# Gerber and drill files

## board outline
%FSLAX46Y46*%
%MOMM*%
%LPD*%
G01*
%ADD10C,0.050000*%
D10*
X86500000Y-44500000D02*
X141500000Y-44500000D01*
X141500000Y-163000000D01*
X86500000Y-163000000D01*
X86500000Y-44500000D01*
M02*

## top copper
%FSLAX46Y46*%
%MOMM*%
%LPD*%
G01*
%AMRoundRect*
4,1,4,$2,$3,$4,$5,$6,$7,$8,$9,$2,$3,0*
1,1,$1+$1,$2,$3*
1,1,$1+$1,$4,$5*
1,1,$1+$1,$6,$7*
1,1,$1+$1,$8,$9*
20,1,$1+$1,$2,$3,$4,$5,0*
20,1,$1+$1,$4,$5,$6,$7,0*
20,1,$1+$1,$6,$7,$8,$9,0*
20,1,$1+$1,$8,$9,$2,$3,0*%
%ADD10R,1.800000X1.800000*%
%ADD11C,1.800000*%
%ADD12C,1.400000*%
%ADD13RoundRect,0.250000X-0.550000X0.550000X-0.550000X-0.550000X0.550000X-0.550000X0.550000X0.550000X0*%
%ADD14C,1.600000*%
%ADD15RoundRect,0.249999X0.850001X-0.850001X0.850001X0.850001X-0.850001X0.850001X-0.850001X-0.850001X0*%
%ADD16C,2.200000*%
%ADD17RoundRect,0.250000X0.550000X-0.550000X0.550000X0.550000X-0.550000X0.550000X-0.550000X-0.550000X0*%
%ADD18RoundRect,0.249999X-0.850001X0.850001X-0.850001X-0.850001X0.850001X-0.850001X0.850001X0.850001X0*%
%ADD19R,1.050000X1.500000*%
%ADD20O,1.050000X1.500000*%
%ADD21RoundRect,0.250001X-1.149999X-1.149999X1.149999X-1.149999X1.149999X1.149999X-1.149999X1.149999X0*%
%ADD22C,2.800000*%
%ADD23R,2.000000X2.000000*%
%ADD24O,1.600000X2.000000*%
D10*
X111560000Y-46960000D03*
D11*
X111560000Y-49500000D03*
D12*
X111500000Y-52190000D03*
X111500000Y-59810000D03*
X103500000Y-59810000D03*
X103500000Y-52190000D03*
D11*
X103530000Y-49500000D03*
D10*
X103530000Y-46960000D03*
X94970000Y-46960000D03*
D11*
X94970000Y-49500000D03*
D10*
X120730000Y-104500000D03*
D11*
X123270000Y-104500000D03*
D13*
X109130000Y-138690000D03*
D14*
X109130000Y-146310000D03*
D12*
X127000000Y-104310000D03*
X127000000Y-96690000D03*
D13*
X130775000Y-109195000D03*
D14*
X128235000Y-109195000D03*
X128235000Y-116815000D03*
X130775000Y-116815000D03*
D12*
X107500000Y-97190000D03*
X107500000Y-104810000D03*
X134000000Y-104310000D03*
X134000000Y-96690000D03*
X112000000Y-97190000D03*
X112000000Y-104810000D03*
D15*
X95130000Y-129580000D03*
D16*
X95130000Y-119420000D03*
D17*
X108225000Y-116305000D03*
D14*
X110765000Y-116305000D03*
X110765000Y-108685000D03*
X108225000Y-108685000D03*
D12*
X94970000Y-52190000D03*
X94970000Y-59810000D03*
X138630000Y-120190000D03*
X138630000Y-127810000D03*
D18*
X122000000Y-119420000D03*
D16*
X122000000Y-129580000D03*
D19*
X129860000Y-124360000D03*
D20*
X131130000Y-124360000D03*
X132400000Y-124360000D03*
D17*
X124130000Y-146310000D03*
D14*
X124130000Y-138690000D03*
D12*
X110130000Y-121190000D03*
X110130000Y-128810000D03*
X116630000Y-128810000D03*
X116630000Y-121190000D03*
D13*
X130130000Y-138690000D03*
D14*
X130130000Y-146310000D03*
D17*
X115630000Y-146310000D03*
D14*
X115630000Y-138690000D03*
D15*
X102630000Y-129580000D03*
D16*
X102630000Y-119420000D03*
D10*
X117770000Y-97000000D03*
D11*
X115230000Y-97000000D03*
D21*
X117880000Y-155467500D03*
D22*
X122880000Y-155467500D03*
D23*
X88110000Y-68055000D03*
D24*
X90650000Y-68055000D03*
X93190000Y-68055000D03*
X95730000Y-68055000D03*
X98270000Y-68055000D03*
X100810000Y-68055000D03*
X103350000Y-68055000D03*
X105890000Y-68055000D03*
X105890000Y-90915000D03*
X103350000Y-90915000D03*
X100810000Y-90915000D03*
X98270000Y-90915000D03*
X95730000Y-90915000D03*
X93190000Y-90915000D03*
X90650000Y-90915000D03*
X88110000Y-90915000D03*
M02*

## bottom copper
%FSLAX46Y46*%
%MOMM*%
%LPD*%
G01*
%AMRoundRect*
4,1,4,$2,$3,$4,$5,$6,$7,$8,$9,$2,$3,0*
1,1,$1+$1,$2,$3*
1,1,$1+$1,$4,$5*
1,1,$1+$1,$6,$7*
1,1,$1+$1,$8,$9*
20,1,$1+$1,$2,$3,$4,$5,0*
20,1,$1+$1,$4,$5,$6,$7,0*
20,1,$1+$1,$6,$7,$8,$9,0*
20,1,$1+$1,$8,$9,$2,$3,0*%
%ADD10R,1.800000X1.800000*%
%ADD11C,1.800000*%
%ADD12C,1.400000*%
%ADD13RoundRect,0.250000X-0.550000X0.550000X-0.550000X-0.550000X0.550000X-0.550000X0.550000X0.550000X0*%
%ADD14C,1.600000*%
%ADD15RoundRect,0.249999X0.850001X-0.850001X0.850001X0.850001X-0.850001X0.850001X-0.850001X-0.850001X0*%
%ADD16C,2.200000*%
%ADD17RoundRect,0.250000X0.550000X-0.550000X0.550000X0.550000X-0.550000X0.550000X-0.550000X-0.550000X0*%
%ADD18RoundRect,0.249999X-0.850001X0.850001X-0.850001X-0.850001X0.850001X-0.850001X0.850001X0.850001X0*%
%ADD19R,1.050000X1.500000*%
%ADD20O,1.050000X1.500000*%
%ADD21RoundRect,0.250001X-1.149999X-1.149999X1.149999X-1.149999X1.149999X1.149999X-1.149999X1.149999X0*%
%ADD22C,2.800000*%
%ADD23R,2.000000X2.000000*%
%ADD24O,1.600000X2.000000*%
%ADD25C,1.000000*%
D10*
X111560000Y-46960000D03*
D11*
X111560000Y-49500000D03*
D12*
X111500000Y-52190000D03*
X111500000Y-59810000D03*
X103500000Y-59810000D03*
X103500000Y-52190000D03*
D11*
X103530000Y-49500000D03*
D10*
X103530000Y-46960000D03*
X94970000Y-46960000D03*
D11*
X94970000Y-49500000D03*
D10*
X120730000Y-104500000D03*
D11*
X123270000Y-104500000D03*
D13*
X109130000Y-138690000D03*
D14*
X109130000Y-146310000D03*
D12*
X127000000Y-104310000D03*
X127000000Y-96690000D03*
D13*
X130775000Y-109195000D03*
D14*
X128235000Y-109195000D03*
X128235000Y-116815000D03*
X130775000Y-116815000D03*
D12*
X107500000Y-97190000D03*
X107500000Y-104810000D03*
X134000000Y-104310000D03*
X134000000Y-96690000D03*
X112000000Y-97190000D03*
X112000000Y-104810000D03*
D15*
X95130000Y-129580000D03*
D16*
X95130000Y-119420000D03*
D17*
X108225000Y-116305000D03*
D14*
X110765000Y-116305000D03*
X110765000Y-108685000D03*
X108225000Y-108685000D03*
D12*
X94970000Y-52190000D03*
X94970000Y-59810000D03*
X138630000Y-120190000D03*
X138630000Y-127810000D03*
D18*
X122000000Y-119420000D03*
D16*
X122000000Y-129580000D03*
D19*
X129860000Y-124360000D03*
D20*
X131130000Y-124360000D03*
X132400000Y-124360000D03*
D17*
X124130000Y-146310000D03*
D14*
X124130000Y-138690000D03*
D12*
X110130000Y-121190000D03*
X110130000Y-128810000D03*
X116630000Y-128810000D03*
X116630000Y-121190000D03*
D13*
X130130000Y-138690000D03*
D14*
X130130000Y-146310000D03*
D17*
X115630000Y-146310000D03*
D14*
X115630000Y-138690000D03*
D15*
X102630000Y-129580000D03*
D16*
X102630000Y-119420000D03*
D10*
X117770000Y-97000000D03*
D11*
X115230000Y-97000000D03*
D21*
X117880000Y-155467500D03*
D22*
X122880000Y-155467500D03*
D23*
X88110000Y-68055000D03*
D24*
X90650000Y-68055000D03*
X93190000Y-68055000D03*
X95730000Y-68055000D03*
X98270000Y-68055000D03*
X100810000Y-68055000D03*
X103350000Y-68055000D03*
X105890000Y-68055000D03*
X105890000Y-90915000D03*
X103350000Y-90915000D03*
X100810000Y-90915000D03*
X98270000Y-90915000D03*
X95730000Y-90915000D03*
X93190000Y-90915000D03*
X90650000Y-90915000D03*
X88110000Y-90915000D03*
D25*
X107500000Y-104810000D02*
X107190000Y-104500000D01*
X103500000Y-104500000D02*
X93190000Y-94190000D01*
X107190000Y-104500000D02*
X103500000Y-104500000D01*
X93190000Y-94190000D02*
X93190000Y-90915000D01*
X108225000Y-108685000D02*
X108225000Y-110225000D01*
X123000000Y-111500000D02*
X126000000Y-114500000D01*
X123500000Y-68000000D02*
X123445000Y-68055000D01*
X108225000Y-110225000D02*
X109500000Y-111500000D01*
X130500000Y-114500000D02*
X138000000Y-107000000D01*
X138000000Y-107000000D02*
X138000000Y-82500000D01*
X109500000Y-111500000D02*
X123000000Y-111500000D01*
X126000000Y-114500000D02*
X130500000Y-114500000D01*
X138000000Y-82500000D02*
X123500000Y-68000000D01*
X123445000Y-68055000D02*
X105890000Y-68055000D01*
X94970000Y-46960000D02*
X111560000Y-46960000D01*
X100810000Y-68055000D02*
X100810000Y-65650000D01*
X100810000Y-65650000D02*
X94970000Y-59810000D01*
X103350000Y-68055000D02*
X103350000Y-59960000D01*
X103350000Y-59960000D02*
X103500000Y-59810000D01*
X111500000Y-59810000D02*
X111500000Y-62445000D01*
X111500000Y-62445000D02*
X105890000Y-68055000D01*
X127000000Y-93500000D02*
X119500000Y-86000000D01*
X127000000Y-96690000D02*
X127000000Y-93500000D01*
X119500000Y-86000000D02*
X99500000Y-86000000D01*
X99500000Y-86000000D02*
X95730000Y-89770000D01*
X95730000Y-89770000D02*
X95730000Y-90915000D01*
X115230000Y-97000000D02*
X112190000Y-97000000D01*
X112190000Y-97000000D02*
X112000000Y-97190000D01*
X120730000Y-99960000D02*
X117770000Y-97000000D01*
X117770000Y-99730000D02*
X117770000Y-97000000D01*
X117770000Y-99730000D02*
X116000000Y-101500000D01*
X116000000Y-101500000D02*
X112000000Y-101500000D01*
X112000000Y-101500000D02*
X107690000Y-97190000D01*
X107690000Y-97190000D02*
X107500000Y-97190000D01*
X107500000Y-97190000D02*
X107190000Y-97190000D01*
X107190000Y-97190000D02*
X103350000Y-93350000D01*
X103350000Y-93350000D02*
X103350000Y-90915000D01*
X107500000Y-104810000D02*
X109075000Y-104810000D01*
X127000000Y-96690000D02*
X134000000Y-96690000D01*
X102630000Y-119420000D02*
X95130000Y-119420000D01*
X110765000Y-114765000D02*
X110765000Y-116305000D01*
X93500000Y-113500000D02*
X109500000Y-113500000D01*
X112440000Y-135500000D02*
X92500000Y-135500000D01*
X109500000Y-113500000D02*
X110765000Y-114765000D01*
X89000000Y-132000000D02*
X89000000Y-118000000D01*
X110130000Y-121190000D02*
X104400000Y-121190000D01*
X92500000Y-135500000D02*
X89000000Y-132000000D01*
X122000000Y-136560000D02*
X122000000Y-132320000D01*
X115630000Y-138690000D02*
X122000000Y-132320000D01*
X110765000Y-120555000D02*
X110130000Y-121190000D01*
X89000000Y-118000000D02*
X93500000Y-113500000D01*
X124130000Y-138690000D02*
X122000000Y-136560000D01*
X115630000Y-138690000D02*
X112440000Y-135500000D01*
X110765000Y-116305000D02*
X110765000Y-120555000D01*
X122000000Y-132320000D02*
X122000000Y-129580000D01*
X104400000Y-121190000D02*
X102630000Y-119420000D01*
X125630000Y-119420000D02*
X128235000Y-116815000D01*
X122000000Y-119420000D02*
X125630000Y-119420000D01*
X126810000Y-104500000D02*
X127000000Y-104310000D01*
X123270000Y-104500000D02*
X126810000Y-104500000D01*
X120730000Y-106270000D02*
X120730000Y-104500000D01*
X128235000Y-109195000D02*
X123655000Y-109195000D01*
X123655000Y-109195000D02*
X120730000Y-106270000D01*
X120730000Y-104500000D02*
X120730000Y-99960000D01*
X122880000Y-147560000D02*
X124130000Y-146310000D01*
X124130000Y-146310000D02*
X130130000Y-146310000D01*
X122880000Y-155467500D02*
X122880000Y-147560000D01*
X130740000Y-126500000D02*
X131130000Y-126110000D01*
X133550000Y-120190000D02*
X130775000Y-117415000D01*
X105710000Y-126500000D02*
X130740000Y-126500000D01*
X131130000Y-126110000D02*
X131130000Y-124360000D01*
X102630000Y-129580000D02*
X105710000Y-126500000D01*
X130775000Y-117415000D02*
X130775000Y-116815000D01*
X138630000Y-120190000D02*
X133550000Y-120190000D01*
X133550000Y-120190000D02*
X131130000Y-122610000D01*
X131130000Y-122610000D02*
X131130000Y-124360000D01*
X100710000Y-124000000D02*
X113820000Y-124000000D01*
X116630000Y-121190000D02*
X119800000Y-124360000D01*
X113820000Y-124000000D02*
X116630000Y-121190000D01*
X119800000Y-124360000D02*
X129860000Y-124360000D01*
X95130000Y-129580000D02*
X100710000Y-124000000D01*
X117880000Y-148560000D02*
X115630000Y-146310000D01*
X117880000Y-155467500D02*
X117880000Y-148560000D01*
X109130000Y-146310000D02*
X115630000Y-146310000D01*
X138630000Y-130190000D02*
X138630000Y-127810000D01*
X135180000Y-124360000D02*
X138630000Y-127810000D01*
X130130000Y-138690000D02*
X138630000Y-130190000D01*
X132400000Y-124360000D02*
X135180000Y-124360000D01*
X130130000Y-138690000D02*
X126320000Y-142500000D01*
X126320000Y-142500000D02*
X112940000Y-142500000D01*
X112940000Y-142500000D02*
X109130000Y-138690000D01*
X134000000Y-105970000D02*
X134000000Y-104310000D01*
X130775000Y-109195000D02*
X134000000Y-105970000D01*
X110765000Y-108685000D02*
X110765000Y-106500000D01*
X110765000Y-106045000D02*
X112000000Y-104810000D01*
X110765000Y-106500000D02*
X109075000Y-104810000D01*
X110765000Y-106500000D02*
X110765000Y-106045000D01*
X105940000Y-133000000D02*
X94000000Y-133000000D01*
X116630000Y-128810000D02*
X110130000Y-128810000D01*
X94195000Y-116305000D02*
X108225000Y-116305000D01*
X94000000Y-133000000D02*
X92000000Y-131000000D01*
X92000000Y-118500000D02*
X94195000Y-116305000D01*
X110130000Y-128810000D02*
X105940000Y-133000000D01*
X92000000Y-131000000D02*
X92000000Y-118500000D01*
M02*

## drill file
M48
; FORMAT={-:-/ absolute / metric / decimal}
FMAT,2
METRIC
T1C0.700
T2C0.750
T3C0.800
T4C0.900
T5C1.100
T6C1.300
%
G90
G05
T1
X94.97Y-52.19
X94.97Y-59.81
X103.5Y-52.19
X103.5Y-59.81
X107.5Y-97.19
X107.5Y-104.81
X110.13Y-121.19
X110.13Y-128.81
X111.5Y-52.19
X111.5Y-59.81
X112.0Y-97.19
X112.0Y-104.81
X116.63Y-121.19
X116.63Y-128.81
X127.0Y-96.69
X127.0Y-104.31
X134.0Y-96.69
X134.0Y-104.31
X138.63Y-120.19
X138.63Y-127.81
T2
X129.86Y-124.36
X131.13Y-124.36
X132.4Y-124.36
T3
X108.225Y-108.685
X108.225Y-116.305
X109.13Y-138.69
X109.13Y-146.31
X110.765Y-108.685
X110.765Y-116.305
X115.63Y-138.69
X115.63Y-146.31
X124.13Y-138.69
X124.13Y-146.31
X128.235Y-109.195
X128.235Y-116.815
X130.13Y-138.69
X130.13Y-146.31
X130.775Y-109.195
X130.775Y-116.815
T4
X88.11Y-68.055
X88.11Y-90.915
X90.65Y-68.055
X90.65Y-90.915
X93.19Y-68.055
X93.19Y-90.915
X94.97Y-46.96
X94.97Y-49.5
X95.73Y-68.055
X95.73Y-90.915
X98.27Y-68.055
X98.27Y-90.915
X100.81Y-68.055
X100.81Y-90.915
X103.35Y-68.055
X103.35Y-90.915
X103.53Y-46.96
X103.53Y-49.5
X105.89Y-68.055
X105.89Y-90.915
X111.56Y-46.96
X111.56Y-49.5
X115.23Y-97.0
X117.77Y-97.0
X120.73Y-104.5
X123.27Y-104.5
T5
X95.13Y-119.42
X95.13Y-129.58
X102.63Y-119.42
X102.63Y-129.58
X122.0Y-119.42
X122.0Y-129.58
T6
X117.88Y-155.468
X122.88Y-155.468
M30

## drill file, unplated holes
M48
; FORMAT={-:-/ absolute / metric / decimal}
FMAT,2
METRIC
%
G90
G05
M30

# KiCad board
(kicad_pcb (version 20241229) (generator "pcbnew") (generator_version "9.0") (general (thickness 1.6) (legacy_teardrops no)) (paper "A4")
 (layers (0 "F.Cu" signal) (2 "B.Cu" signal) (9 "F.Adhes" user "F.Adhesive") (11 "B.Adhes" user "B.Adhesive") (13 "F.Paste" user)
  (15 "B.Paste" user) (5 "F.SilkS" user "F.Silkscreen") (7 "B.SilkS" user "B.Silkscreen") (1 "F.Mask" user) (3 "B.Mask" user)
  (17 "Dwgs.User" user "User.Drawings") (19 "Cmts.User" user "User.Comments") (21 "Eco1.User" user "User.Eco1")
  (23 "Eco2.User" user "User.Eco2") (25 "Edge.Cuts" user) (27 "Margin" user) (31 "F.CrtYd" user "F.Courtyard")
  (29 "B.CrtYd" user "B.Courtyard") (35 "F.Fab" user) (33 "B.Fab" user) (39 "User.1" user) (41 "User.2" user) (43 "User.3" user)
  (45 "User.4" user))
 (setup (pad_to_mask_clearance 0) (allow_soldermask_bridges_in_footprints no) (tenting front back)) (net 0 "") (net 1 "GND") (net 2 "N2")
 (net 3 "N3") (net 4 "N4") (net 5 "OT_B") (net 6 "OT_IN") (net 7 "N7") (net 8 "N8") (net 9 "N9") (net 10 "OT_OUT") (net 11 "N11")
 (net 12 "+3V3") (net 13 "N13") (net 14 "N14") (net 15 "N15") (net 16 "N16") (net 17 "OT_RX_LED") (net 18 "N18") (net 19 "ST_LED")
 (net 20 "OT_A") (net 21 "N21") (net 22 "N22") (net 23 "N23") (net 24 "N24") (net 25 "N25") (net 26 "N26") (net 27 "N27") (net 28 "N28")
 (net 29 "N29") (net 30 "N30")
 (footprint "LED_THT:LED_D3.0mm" (layer "F.Cu") (at 94.97 46.96 -90)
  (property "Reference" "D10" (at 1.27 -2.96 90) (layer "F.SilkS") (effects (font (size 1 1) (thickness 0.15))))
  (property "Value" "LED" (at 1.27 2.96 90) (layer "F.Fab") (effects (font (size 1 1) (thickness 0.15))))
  (pad "1" thru_hole rect (at 0 0 270) (size 1.8 1.8) (drill 0.9) (layers "*.Cu" "*.Mask") (remove_unused_layers no) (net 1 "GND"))
  (pad "2" thru_hole circle (at 2.54 0 270) (size 1.8 1.8) (drill 0.9) (layers "*.Cu" "*.Mask") (remove_unused_layers no) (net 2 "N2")))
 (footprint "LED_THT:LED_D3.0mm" (layer "F.Cu") (at 120.73 104.5)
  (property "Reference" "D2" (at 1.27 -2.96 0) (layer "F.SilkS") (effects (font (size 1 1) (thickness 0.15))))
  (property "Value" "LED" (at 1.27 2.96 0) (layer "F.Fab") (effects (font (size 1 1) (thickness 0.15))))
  (pad "1" thru_hole rect (at 0 0) (size 1.8 1.8) (drill 0.9) (layers "*.Cu" "*.Mask") (remove_unused_layers no) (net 1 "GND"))
  (pad "2" thru_hole circle (at 2.54 0) (size 1.8 1.8) (drill 0.9) (layers "*.Cu" "*.Mask") (remove_unused_layers no) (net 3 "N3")))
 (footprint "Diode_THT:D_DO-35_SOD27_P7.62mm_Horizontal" (layer "F.Cu") (at 109.13 138.69 -90)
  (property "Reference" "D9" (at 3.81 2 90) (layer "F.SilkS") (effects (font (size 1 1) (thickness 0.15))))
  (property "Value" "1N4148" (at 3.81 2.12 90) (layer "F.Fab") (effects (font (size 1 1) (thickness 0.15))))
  (pad "1" thru_hole roundrect (at 0 0 270) (size 1.6 1.6) (drill 0.8) (layers "*.Cu" "*.Mask") (remove_unused_layers no)
   (roundrect_rratio 0.15625) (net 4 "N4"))
  (pad "2" thru_hole circle (at 7.62 0 270) (size 1.6 1.6) (drill 0.8) (layers "*.Cu" "*.Mask") (remove_unused_layers no) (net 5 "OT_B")))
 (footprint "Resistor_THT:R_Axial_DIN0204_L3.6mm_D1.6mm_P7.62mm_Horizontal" (layer "F.Cu") (at 127 104.31 90)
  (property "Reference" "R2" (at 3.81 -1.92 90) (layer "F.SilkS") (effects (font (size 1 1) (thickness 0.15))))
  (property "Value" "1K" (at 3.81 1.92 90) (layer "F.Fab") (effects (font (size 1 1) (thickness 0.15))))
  (pad "1" thru_hole circle (at 0 0 90) (size 1.4 1.4) (drill 0.7) (layers "*.Cu" "*.Mask") (remove_unused_layers no) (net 3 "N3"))
  (pad "2" thru_hole circle (at 7.62 0 90) (size 1.4 1.4) (drill 0.7) (layers "*.Cu" "*.Mask") (remove_unused_layers no) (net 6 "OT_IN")))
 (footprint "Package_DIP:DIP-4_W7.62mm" (layer "F.Cu") (at 130.775 109.195 -90)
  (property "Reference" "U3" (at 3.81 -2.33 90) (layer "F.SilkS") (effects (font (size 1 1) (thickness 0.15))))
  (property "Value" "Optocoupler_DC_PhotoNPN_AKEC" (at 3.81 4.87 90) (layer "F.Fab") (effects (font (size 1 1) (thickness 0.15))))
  (pad "1" thru_hole roundrect (at 0 0 270) (size 1.6 1.6) (drill 0.8) (layers "*.Cu" "*.Mask") (remove_unused_layers no)
   (roundrect_rratio 0.15625) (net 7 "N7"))
  (pad "2" thru_hole circle (at 0 2.54 270) (size 1.6 1.6) (drill 0.8) (layers "*.Cu" "*.Mask") (remove_unused_layers no) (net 1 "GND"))
  (pad "3" thru_hole circle (at 7.62 2.54 270) (size 1.6 1.6) (drill 0.8) (layers "*.Cu" "*.Mask") (remove_unused_layers no) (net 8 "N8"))
  (pad "4" thru_hole circle (at 7.62 0 270) (size 1.6 1.6) (drill 0.8) (layers "*.Cu" "*.Mask") (remove_unused_layers no) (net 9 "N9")))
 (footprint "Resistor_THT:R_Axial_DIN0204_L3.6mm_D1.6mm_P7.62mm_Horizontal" (layer "F.Cu") (at 107.5 97.19 -90)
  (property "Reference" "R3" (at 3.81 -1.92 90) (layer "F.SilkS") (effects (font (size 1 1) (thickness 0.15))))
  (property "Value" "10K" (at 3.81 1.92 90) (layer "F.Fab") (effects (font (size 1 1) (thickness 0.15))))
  (pad "1" thru_hole circle (at 0 0 270) (size 1.4 1.4) (drill 0.7) (layers "*.Cu" "*.Mask") (remove_unused_layers no) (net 1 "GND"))
  (pad "2" thru_hole circle (at 7.62 0 270) (size 1.4 1.4) (drill 0.7) (layers "*.Cu" "*.Mask") (remove_unused_layers no) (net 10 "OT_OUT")))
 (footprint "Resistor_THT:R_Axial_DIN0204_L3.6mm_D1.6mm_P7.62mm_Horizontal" (layer "F.Cu") (at 134 104.31 90)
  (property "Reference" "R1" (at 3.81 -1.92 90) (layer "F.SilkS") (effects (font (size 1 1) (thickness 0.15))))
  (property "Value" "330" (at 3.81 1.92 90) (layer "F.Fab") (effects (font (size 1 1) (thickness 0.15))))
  (pad "1" thru_hole circle (at 0 0 90) (size 1.4 1.4) (drill 0.7) (layers "*.Cu" "*.Mask") (remove_unused_layers no) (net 7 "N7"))
  (pad "2" thru_hole circle (at 7.62 0 90) (size 1.4 1.4) (drill 0.7) (layers "*.Cu" "*.Mask") (remove_unused_layers no) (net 6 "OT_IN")))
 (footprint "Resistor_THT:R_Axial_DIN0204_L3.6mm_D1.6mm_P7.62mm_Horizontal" (layer "F.Cu") (at 111.5 52.19 -90)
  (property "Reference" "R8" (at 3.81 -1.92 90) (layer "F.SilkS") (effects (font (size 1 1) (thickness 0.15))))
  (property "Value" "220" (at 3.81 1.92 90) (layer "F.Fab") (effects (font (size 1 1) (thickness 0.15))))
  (pad "1" thru_hole circle (at 0 0 270) (size 1.4 1.4) (drill 0.7) (layers "*.Cu" "*.Mask") (remove_unused_layers no) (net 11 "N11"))
  (pad "2" thru_hole circle (at 7.62 0 270) (size 1.4 1.4) (drill 0.7) (layers "*.Cu" "*.Mask") (remove_unused_layers no) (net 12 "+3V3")))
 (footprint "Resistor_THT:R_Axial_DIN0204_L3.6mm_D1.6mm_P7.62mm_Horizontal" (layer "F.Cu") (at 112 97.19 -90)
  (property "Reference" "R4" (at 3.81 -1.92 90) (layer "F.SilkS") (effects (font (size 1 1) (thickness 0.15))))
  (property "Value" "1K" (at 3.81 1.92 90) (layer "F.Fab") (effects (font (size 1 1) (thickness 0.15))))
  (pad "1" thru_hole circle (at 0 0 270) (size 1.4 1.4) (drill 0.7) (layers "*.Cu" "*.Mask") (remove_unused_layers no) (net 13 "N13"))
  (pad "2" thru_hole circle (at 7.62 0 270) (size 1.4 1.4) (drill 0.7) (layers "*.Cu" "*.Mask") (remove_unused_layers no) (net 10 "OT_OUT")))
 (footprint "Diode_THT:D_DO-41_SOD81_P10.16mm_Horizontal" (layer "F.Cu") (at 95.13 129.58 90)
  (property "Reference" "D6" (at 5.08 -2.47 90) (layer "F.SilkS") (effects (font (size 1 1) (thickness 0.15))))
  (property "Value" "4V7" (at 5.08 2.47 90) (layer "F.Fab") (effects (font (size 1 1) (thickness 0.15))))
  (pad "1" thru_hole roundrect (at 0 0 90) (size 2.2 2.2) (drill 1.1) (layers "*.Cu" "*.Mask") (remove_unused_layers no)
   (roundrect_rratio 0.113636) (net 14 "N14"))
  (pad "2" thru_hole circle (at 10.16 0 90) (size 2.2 2.2) (drill 1.1) (layers "*.Cu" "*.Mask") (remove_unused_layers no) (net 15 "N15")))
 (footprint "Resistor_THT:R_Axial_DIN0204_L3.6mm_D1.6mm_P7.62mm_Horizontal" (layer "F.Cu") (at 103.5 52.19 -90)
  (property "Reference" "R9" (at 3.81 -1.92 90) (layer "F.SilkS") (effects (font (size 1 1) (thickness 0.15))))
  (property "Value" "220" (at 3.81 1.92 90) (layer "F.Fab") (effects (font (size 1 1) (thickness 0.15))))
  (pad "1" thru_hole circle (at 0 0 270) (size 1.4 1.4) (drill 0.7) (layers "*.Cu" "*.Mask") (remove_unused_layers no) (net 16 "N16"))
  (pad "2" thru_hole circle (at 7.62 0 270) (size 1.4 1.4) (drill 0.7) (layers "*.Cu" "*.Mask") (remove_unused_layers no)
   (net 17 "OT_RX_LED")))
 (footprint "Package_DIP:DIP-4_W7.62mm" (layer "F.Cu") (at 108.225 116.305 90)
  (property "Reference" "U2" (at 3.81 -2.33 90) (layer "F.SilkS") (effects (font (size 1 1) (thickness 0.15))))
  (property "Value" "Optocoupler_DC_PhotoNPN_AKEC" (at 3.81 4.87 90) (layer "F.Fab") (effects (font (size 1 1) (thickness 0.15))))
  (pad "1" thru_hole roundrect (at 0 0 90) (size 1.6 1.6) (drill 0.8) (layers "*.Cu" "*.Mask") (remove_unused_layers no)
   (roundrect_rratio 0.15625) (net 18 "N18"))
  (pad "2" thru_hole circle (at 0 2.54 90) (size 1.6 1.6) (drill 0.8) (layers "*.Cu" "*.Mask") (remove_unused_layers no) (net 15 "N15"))
  (pad "3" thru_hole circle (at 7.62 2.54 90) (size 1.6 1.6) (drill 0.8) (layers "*.Cu" "*.Mask") (remove_unused_layers no)
   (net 10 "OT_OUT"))
  (pad "4" thru_hole circle (at 7.62 0 90) (size 1.6 1.6) (drill 0.8) (layers "*.Cu" "*.Mask") (remove_unused_layers no) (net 12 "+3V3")))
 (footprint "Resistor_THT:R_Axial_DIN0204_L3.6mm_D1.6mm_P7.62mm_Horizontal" (layer "F.Cu") (at 94.97 52.19 -90)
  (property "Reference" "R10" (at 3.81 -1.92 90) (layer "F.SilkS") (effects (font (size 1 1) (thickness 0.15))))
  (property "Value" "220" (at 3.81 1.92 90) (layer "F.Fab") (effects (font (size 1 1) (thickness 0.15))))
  (pad "1" thru_hole circle (at 0 0 270) (size 1.4 1.4) (drill 0.7) (layers "*.Cu" "*.Mask") (remove_unused_layers no) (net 2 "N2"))
  (pad "2" thru_hole circle (at 7.62 0 270) (size 1.4 1.4) (drill 0.7) (layers "*.Cu" "*.Mask") (remove_unused_layers no) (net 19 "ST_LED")))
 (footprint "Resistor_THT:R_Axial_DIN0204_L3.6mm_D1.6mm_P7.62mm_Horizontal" (layer "F.Cu") (at 138.63 120.19 -90)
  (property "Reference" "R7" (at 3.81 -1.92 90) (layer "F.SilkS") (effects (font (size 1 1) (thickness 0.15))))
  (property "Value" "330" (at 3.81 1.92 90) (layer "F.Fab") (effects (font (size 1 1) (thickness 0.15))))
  (pad "1" thru_hole circle (at 0 0 270) (size 1.4 1.4) (drill 0.7) (layers "*.Cu" "*.Mask") (remove_unused_layers no) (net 9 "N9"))
  (pad "2" thru_hole circle (at 7.62 0 270) (size 1.4 1.4) (drill 0.7) (layers "*.Cu" "*.Mask") (remove_unused_layers no) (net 4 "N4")))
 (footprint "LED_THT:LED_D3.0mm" (layer "F.Cu") (at 111.56 46.96 -90)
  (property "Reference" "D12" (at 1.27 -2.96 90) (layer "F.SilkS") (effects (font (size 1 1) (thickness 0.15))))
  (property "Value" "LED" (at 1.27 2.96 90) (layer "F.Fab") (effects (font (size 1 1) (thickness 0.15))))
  (pad "1" thru_hole rect (at 0 0 270) (size 1.8 1.8) (drill 0.9) (layers "*.Cu" "*.Mask") (remove_unused_layers no) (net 1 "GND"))
  (pad "2" thru_hole circle (at 2.54 0 270) (size 1.8 1.8) (drill 0.9) (layers "*.Cu" "*.Mask") (remove_unused_layers no) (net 11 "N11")))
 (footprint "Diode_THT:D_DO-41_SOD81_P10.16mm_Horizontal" (layer "F.Cu") (at 122 119.42 -90)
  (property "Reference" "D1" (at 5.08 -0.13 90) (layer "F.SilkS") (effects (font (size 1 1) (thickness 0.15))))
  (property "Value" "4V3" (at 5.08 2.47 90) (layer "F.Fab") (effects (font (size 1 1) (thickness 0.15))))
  (pad "1" thru_hole roundrect (at 0 0 270) (size 2.2 2.2) (drill 1.1) (layers "*.Cu" "*.Mask") (remove_unused_layers no)
   (roundrect_rratio 0.113636) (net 8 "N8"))
  (pad "2" thru_hole circle (at 10.16 0 270) (size 2.2 2.2) (drill 1.1) (layers "*.Cu" "*.Mask") (remove_unused_layers no) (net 15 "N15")))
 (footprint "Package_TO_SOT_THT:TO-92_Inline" (layer "F.Cu") (at 129.86 124.36)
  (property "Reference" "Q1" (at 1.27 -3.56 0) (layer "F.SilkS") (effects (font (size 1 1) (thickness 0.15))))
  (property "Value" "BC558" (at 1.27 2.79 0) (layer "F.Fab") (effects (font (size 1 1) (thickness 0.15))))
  (pad "1" thru_hole rect (at 0 0) (size 1.05 1.5) (drill 0.75) (layers "*.Cu" "*.Mask") (remove_unused_layers no) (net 14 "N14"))
  (pad "2" thru_hole oval (at 1.27 0) (size 1.05 1.5) (drill 0.75) (layers "*.Cu" "*.Mask") (remove_unused_layers no) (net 9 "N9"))
  (pad "3" thru_hole oval (at 2.54 0) (size 1.05 1.5) (drill 0.75) (layers "*.Cu" "*.Mask") (remove_unused_layers no) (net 4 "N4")))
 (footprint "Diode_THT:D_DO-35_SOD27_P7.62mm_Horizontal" (layer "F.Cu") (at 124.13 146.31 90)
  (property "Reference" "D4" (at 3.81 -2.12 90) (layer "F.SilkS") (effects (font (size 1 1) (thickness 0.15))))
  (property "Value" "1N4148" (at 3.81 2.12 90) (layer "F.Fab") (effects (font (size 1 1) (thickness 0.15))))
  (pad "1" thru_hole roundrect (at 0 0 90) (size 1.6 1.6) (drill 0.8) (layers "*.Cu" "*.Mask") (remove_unused_layers no)
   (roundrect_rratio 0.15625) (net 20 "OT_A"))
  (pad "2" thru_hole circle (at 7.62 0 90) (size 1.6 1.6) (drill 0.8) (layers "*.Cu" "*.Mask") (remove_unused_layers no) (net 15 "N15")))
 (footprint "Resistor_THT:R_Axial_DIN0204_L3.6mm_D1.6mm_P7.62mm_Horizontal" (layer "F.Cu") (at 110.13 121.19 -90)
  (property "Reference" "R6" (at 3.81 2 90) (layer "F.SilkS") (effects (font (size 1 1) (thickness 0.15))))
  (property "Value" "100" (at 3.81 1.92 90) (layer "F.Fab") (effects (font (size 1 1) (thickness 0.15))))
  (pad "1" thru_hole circle (at 0 0 270) (size 1.4 1.4) (drill 0.7) (layers "*.Cu" "*.Mask") (remove_unused_layers no) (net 15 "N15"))
  (pad "2" thru_hole circle (at 7.62 0 270) (size 1.4 1.4) (drill 0.7) (layers "*.Cu" "*.Mask") (remove_unused_layers no) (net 18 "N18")))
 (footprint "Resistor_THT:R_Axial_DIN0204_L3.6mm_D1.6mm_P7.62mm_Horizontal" (layer "F.Cu") (at 116.63 128.81 90)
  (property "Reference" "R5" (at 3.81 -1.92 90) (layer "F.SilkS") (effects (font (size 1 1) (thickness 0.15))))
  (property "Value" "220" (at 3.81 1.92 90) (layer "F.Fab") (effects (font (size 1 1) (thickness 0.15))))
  (pad "1" thru_hole circle (at 0 0 90) (size 1.4 1.4) (drill 0.7) (layers "*.Cu" "*.Mask") (remove_unused_layers no) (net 18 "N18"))
  (pad "2" thru_hole circle (at 7.62 0 90) (size 1.4 1.4) (drill 0.7) (layers "*.Cu" "*.Mask") (remove_unused_layers no) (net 14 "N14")))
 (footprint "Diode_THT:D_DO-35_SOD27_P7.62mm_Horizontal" (layer "F.Cu") (at 130.13 138.69 -90)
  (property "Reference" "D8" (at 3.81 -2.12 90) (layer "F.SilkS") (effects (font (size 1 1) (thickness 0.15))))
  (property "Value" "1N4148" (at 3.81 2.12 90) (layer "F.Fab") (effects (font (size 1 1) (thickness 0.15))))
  (pad "1" thru_hole roundrect (at 0 0 270) (size 1.6 1.6) (drill 0.8) (layers "*.Cu" "*.Mask") (remove_unused_layers no)
   (roundrect_rratio 0.15625) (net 4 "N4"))
  (pad "2" thru_hole circle (at 7.62 0 270) (size 1.6 1.6) (drill 0.8) (layers "*.Cu" "*.Mask") (remove_unused_layers no) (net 20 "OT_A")))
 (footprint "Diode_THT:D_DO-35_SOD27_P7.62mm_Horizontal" (layer "F.Cu") (at 115.63 146.31 90)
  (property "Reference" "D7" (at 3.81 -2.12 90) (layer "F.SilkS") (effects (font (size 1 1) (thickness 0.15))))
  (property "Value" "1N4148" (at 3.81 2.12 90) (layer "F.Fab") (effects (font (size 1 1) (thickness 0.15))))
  (pad "1" thru_hole roundrect (at 0 0 90) (size 1.6 1.6) (drill 0.8) (layers "*.Cu" "*.Mask") (remove_unused_layers no)
   (roundrect_rratio 0.15625) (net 5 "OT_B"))
  (pad "2" thru_hole circle (at 7.62 0 90) (size 1.6 1.6) (drill 0.8) (layers "*.Cu" "*.Mask") (remove_unused_layers no) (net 15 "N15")))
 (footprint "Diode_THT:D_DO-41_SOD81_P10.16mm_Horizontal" (layer "F.Cu") (at 102.63 129.58 90)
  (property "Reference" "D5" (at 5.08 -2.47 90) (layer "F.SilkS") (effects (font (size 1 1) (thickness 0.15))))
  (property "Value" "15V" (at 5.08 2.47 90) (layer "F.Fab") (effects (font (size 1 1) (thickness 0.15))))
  (pad "1" thru_hole roundrect (at 0 0 90) (size 2.2 2.2) (drill 1.1) (layers "*.Cu" "*.Mask") (remove_unused_layers no)
   (roundrect_rratio 0.113636) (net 9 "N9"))
  (pad "2" thru_hole circle (at 10.16 0 90) (size 2.2 2.2) (drill 1.1) (layers "*.Cu" "*.Mask") (remove_unused_layers no) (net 15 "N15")))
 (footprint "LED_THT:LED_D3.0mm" (layer "F.Cu") (at 117.77 97 180)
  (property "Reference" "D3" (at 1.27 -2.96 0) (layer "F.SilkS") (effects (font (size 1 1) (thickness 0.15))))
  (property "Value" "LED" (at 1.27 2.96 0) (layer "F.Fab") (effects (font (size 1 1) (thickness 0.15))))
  (pad "1" thru_hole rect (at 0 0 180) (size 1.8 1.8) (drill 0.9) (layers "*.Cu" "*.Mask") (remove_unused_layers no) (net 1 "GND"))
  (pad "2" thru_hole circle (at 2.54 0 180) (size 1.8 1.8) (drill 0.9) (layers "*.Cu" "*.Mask") (remove_unused_layers no) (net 13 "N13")))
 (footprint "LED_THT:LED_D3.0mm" (layer "F.Cu") (at 103.53 46.96 -90)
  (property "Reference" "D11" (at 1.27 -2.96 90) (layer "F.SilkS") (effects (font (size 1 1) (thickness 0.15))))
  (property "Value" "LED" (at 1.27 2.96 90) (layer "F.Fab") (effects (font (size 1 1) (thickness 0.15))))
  (pad "1" thru_hole rect (at 0 0 270) (size 1.8 1.8) (drill 0.9) (layers "*.Cu" "*.Mask") (remove_unused_layers no) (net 1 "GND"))
  (pad "2" thru_hole circle (at 2.54 0 270) (size 1.8 1.8) (drill 0.9) (layers "*.Cu" "*.Mask") (remove_unused_layers no) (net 16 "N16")))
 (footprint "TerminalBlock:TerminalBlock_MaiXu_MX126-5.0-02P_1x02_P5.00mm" (layer "F.Cu") (at 117.88 155.4675)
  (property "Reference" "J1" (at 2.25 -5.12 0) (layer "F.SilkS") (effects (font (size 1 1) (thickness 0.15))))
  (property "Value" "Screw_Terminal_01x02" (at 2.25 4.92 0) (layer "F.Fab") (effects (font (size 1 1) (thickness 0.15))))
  (pad "1" thru_hole roundrect (at 0 0) (size 2.8 2.8) (drill 1.3) (layers "*.Cu" "*.Mask") (remove_unused_layers no)
   (roundrect_rratio 0.089286) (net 5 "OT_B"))
  (pad "2" thru_hole circle (at 5 0) (size 2.8 2.8) (drill 1.3) (layers "*.Cu" "*.Mask") (remove_unused_layers no) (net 20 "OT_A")))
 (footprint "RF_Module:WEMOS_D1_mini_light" (layer "B.Cu") (at 88.11 68.055 -90)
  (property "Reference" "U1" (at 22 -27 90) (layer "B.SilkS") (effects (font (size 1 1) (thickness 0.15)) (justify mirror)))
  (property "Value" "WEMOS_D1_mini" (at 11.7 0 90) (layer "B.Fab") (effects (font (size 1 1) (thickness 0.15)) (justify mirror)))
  (pad "1" thru_hole rect (at 0 0 270) (size 2 2) (drill 0.9) (layers "*.Cu" "*.Mask") (remove_unused_layers no) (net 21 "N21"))
  (pad "2" thru_hole oval (at 0 -2.54 270) (size 2 1.6) (drill 0.9) (layers "*.Cu" "*.Mask") (remove_unused_layers no) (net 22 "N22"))
  (pad "3" thru_hole oval (at 0 -5.08 270) (size 2 1.6) (drill 0.9) (layers "*.Cu" "*.Mask") (remove_unused_layers no) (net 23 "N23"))
  (pad "4" thru_hole oval (at 0 -7.62 270) (size 2 1.6) (drill 0.9) (layers "*.Cu" "*.Mask") (remove_unused_layers no) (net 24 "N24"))
  (pad "5" thru_hole oval (at 0 -10.16 270) (size 2 1.6) (drill 0.9) (layers "*.Cu" "*.Mask") (remove_unused_layers no) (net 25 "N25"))
  (pad "6" thru_hole oval (at 0 -12.7 270) (size 2 1.6) (drill 0.9) (layers "*.Cu" "*.Mask") (remove_unused_layers no) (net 19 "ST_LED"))
  (pad "7" thru_hole oval (at 0 -15.24 270) (size 2 1.6) (drill 0.9) (layers "*.Cu" "*.Mask") (remove_unused_layers no) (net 17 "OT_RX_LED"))
  (pad "8" thru_hole oval (at 0 -17.78 270) (size 2 1.6) (drill 0.9) (layers "*.Cu" "*.Mask") (remove_unused_layers no) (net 12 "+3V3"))
  (pad "9" thru_hole oval (at 22.86 -17.78 270) (size 2 1.6) (drill 0.9) (layers "*.Cu" "*.Mask") (remove_unused_layers no) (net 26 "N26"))
  (pad "10" thru_hole oval (at 22.86 -15.24 270) (size 2 1.6) (drill 0.9) (layers "*.Cu" "*.Mask") (remove_unused_layers no) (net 1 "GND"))
  (pad "11" thru_hole oval (at 22.86 -12.7 270) (size 2 1.6) (drill 0.9) (layers "*.Cu" "*.Mask") (remove_unused_layers no) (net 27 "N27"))
  (pad "12" thru_hole oval (at 22.86 -10.16 270) (size 2 1.6) (drill 0.9) (layers "*.Cu" "*.Mask") (remove_unused_layers no) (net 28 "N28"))
  (pad "13" thru_hole oval (at 22.86 -7.62 270) (size 2 1.6) (drill 0.9) (layers "*.Cu" "*.Mask") (remove_unused_layers no) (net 6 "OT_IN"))
  (pad "14" thru_hole oval (at 22.86 -5.08 270) (size 2 1.6) (drill 0.9) (layers "*.Cu" "*.Mask") (remove_unused_layers no)
   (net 10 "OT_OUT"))
  (pad "15" thru_hole oval (at 22.86 -2.54 270) (size 2 1.6) (drill 0.9) (layers "*.Cu" "*.Mask") (remove_unused_layers no) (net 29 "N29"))
  (pad "16" thru_hole oval (at 22.86 0 270) (size 2 1.6) (drill 0.9) (layers "*.Cu" "*.Mask") (remove_unused_layers no) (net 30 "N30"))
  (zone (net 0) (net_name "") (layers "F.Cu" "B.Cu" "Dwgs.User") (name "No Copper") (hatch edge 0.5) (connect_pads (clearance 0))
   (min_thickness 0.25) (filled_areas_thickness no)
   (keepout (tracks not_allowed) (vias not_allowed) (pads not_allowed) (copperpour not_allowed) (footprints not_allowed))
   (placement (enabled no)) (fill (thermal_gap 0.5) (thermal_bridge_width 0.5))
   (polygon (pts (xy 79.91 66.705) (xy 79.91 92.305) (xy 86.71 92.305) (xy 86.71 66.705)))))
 (gr_rect (start 86.5 44.5) (end 141.5 163) (stroke (width 0.05) (type default)) (fill no) (layer "Edge.Cuts"))
 (segment (start 102.63 119.42) (end 95.13 119.42) (width 1) (layer "B.Cu") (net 15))
 (segment (start 110.765 114.765) (end 110.765 116.305) (width 1) (layer "B.Cu") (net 15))
 (segment (start 93.5 113.5) (end 109.5 113.5) (width 1) (layer "B.Cu") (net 15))
 (segment (start 112.44 135.5) (end 92.5 135.5) (width 1) (layer "B.Cu") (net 15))
 (segment (start 109.5 113.5) (end 110.765 114.765) (width 1) (layer "B.Cu") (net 15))
 (segment (start 89 132) (end 89 118) (width 1) (layer "B.Cu") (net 15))
 (segment (start 110.13 121.19) (end 104.4 121.19) (width 1) (layer "B.Cu") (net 15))
 (segment (start 92.5 135.5) (end 89 132) (width 1) (layer "B.Cu") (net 15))
 (segment (start 122 136.56) (end 122 132.32) (width 1) (layer "B.Cu") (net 15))
 (segment (start 115.63 138.69) (end 122 132.32) (width 1) (layer "B.Cu") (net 15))
 (segment (start 110.765 120.555) (end 110.13 121.19) (width 1) (layer "B.Cu") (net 15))
 (segment (start 89 118) (end 93.5 113.5) (width 1) (layer "B.Cu") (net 15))
 (segment (start 124.13 138.69) (end 122 136.56) (width 1) (layer "B.Cu") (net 15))
 (segment (start 115.63 138.69) (end 112.44 135.5) (width 1) (layer "B.Cu") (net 15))
 (segment (start 110.765 116.305) (end 110.765 120.555) (width 1) (layer "B.Cu") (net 15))
 (segment (start 122 132.32) (end 122 129.58) (width 1) (layer "B.Cu") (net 15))
 (segment (start 104.4 121.19) (end 102.63 119.42) (width 1) (layer "B.Cu") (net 15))
 (segment (start 125.63 119.42) (end 128.235 116.815) (width 1) (layer "B.Cu") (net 8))
 (segment (start 122 119.42) (end 125.63 119.42) (width 1) (layer "B.Cu") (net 8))
 (segment (start 126.81 104.5) (end 127 104.31) (width 1) (layer "B.Cu") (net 3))
 (segment (start 123.27 104.5) (end 126.81 104.5) (width 1) (layer "B.Cu") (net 3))
 (segment (start 117.77 99.73) (end 116 101.5) (width 1) (layer "B.Cu") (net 1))
 (segment (start 107.19 97.19) (end 103.35 93.35) (width 1) (layer "B.Cu") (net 1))
 (segment (start 120.73 106.27) (end 120.73 104.5) (width 1) (layer "B.Cu") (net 1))
 (segment (start 120.73 99.96) (end 117.77 97) (width 1) (layer "B.Cu") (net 1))
 (segment (start 128.235 109.195) (end 123.655 109.195) (width 1) (layer "B.Cu") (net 1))
 (segment (start 107.5 97.19) (end 107.19 97.19) (width 1) (layer "B.Cu") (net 1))
 (segment (start 103.35 93.35) (end 103.35 90.915) (width 1) (layer "B.Cu") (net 1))
 (segment (start 123.655 109.195) (end 120.73 106.27) (width 1) (layer "B.Cu") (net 1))
 (segment (start 116 101.5) (end 112 101.5) (width 1) (layer "B.Cu") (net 1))
 (segment (start 117.77 99.73) (end 117.77 97) (width 1) (layer "B.Cu") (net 1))
 (segment (start 112 101.5) (end 107.69 97.19) (width 1) (layer "B.Cu") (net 1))
 (segment (start 107.69 97.19) (end 107.5 97.19) (width 1) (layer "B.Cu") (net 1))
 (segment (start 94.97 46.96) (end 111.56 46.96) (width 1) (layer "B.Cu") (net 1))
 (segment (start 120.73 104.5) (end 120.73 99.96) (width 1) (layer "B.Cu") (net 1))
 (segment (start 115.23 97) (end 112.19 97) (width 1) (layer "B.Cu") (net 13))
 (segment (start 112.19 97) (end 112 97.19) (width 1) (layer "B.Cu") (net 13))
 (segment (start 122.88 147.56) (end 124.13 146.31) (width 1) (layer "B.Cu") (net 20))
 (segment (start 124.13 146.31) (end 130.13 146.31) (width 1) (layer "B.Cu") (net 20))
 (segment (start 122.88 155.4675) (end 122.88 147.56) (width 1) (layer "B.Cu") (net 20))
 (segment (start 130.74 126.5) (end 131.13 126.11) (width 1) (layer "B.Cu") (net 9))
 (segment (start 133.55 120.19) (end 130.775 117.415) (width 1) (layer "B.Cu") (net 9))
 (segment (start 105.71 126.5) (end 130.74 126.5) (width 1) (layer "B.Cu") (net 9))
 (segment (start 131.13 126.11) (end 131.13 124.36) (width 1) (layer "B.Cu") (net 9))
 (segment (start 102.63 129.58) (end 105.71 126.5) (width 1) (layer "B.Cu") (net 9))
 (segment (start 130.775 117.415) (end 130.775 116.815) (width 1) (layer "B.Cu") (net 9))
 (segment (start 138.63 120.19) (end 133.55 120.19) (width 1) (layer "B.Cu") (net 9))
 (segment (start 133.55 120.19) (end 131.13 122.61) (width 1) (layer "B.Cu") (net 9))
 (segment (start 131.13 122.61) (end 131.13 124.36) (width 1) (layer "B.Cu") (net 9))
 (segment (start 100.71 124) (end 113.82 124) (width 1) (layer "B.Cu") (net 14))
 (segment (start 116.63 121.19) (end 119.8 124.36) (width 1) (layer "B.Cu") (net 14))
 (segment (start 113.82 124) (end 116.63 121.19) (width 1) (layer "B.Cu") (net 14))
 (segment (start 119.8 124.36) (end 129.86 124.36) (width 1) (layer "B.Cu") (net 14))
 (segment (start 95.13 129.58) (end 100.71 124) (width 1) (layer "B.Cu") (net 14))
 (segment (start 117.88 148.56) (end 115.63 146.31) (width 1) (layer "B.Cu") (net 5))
 (segment (start 117.88 155.4675) (end 117.88 148.56) (width 1) (layer "B.Cu") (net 5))
 (segment (start 109.13 146.31) (end 115.63 146.31) (width 1) (layer "B.Cu") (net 5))
 (segment (start 138.63 130.19) (end 138.63 127.81) (width 1) (layer "B.Cu") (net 4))
 (segment (start 135.18 124.36) (end 138.63 127.81) (width 1) (layer "B.Cu") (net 4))
 (segment (start 130.13 138.69) (end 138.63 130.19) (width 1) (layer "B.Cu") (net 4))
 (segment (start 132.4 124.36) (end 135.18 124.36) (width 1) (layer "B.Cu") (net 4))
 (segment (start 130.13 138.69) (end 126.32 142.5) (width 1) (layer "B.Cu") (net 4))
 (segment (start 126.32 142.5) (end 112.94 142.5) (width 1) (layer "B.Cu") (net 4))
 (segment (start 112.94 142.5) (end 109.13 138.69) (width 1) (layer "B.Cu") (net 4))
 (segment (start 99.5 86) (end 95.73 89.77) (width 1) (layer "B.Cu") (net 6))
 (segment (start 119.5 86) (end 99.5 86) (width 1) (layer "B.Cu") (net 6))
 (segment (start 127 96.69) (end 127 93.5) (width 1) (layer "B.Cu") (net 6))
 (segment (start 127 93.5) (end 119.5 86) (width 1) (layer "B.Cu") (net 6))
 (segment (start 95.73 89.77) (end 95.73 90.915) (width 1) (layer "B.Cu") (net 6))
 (segment (start 127 96.69) (end 134 96.69) (width 1) (layer "B.Cu") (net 6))
 (segment (start 134 105.97) (end 134 104.31) (width 1) (layer "B.Cu") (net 7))
 (segment (start 130.775 109.195) (end 134 105.97) (width 1) (layer "B.Cu") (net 7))
 (segment (start 93.19 94.19) (end 93.19 90.915) (width 1) (layer "B.Cu") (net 10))
 (segment (start 110.765 108.685) (end 110.765 106.5) (width 1) (layer "B.Cu") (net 10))
 (segment (start 107.5 104.81) (end 107.19 104.5) (width 1) (layer "B.Cu") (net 10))
 (segment (start 110.765 106.045) (end 112 104.81) (width 1) (layer "B.Cu") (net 10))
 (segment (start 107.19 104.5) (end 103.5 104.5) (width 1) (layer "B.Cu") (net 10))
 (segment (start 103.5 104.5) (end 93.19 94.19) (width 1) (layer "B.Cu") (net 10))
 (segment (start 110.765 106.5) (end 109.075 104.81) (width 1) (layer "B.Cu") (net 10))
 (segment (start 107.5 104.81) (end 109.075 104.81) (width 1) (layer "B.Cu") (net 10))
 (segment (start 110.765 106.5) (end 110.765 106.045) (width 1) (layer "B.Cu") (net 10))
 (segment (start 105.94 133) (end 94 133) (width 1) (layer "B.Cu") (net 18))
 (segment (start 116.63 128.81) (end 110.13 128.81) (width 1) (layer "B.Cu") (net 18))
 (segment (start 94.195 116.305) (end 108.225 116.305) (width 1) (layer "B.Cu") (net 18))
 (segment (start 94 133) (end 92 131) (width 1) (layer "B.Cu") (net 18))
 (segment (start 92 118.5) (end 94.195 116.305) (width 1) (layer "B.Cu") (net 18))
 (segment (start 110.13 128.81) (end 105.94 133) (width 1) (layer "B.Cu") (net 18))
 (segment (start 92 131) (end 92 118.5) (width 1) (layer "B.Cu") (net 18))
 (segment (start 126 114.5) (end 130.5 114.5) (width 1) (layer "B.Cu") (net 12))
 (segment (start 111.5 62.445) (end 105.89 68.055) (width 1) (layer "B.Cu") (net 12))
 (segment (start 109.5 111.5) (end 123 111.5) (width 1) (layer "B.Cu") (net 12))
 (segment (start 123 111.5) (end 126 114.5) (width 1) (layer "B.Cu") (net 12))
 (segment (start 123.5 68) (end 123.445 68.055) (width 1) (layer "B.Cu") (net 12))
 (segment (start 138 107) (end 138 82.5) (width 1) (layer "B.Cu") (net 12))
 (segment (start 138 82.5) (end 123.5 68) (width 1) (layer "B.Cu") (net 12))
 (segment (start 123.445 68.055) (end 105.89 68.055) (width 1) (layer "B.Cu") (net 12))
 (segment (start 130.5 114.5) (end 138 107) (width 1) (layer "B.Cu") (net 12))
 (segment (start 108.225 110.225) (end 109.5 111.5) (width 1) (layer "B.Cu") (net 12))
 (segment (start 111.5 59.81) (end 111.5 62.445) (width 1) (layer "B.Cu") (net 12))
 (segment (start 108.225 108.685) (end 108.225 110.225) (width 1) (layer "B.Cu") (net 12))
 (segment (start 103.35 59.96) (end 103.5 59.81) (width 1) (layer "B.Cu") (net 17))
 (segment (start 103.35 68.055) (end 103.35 59.96) (width 1) (layer "B.Cu") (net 17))
 (segment (start 100.81 68.055) (end 100.81 65.65) (width 1) (layer "B.Cu") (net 19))
 (segment (start 100.81 65.65) (end 94.97 59.81) (width 1) (layer "B.Cu") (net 19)))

